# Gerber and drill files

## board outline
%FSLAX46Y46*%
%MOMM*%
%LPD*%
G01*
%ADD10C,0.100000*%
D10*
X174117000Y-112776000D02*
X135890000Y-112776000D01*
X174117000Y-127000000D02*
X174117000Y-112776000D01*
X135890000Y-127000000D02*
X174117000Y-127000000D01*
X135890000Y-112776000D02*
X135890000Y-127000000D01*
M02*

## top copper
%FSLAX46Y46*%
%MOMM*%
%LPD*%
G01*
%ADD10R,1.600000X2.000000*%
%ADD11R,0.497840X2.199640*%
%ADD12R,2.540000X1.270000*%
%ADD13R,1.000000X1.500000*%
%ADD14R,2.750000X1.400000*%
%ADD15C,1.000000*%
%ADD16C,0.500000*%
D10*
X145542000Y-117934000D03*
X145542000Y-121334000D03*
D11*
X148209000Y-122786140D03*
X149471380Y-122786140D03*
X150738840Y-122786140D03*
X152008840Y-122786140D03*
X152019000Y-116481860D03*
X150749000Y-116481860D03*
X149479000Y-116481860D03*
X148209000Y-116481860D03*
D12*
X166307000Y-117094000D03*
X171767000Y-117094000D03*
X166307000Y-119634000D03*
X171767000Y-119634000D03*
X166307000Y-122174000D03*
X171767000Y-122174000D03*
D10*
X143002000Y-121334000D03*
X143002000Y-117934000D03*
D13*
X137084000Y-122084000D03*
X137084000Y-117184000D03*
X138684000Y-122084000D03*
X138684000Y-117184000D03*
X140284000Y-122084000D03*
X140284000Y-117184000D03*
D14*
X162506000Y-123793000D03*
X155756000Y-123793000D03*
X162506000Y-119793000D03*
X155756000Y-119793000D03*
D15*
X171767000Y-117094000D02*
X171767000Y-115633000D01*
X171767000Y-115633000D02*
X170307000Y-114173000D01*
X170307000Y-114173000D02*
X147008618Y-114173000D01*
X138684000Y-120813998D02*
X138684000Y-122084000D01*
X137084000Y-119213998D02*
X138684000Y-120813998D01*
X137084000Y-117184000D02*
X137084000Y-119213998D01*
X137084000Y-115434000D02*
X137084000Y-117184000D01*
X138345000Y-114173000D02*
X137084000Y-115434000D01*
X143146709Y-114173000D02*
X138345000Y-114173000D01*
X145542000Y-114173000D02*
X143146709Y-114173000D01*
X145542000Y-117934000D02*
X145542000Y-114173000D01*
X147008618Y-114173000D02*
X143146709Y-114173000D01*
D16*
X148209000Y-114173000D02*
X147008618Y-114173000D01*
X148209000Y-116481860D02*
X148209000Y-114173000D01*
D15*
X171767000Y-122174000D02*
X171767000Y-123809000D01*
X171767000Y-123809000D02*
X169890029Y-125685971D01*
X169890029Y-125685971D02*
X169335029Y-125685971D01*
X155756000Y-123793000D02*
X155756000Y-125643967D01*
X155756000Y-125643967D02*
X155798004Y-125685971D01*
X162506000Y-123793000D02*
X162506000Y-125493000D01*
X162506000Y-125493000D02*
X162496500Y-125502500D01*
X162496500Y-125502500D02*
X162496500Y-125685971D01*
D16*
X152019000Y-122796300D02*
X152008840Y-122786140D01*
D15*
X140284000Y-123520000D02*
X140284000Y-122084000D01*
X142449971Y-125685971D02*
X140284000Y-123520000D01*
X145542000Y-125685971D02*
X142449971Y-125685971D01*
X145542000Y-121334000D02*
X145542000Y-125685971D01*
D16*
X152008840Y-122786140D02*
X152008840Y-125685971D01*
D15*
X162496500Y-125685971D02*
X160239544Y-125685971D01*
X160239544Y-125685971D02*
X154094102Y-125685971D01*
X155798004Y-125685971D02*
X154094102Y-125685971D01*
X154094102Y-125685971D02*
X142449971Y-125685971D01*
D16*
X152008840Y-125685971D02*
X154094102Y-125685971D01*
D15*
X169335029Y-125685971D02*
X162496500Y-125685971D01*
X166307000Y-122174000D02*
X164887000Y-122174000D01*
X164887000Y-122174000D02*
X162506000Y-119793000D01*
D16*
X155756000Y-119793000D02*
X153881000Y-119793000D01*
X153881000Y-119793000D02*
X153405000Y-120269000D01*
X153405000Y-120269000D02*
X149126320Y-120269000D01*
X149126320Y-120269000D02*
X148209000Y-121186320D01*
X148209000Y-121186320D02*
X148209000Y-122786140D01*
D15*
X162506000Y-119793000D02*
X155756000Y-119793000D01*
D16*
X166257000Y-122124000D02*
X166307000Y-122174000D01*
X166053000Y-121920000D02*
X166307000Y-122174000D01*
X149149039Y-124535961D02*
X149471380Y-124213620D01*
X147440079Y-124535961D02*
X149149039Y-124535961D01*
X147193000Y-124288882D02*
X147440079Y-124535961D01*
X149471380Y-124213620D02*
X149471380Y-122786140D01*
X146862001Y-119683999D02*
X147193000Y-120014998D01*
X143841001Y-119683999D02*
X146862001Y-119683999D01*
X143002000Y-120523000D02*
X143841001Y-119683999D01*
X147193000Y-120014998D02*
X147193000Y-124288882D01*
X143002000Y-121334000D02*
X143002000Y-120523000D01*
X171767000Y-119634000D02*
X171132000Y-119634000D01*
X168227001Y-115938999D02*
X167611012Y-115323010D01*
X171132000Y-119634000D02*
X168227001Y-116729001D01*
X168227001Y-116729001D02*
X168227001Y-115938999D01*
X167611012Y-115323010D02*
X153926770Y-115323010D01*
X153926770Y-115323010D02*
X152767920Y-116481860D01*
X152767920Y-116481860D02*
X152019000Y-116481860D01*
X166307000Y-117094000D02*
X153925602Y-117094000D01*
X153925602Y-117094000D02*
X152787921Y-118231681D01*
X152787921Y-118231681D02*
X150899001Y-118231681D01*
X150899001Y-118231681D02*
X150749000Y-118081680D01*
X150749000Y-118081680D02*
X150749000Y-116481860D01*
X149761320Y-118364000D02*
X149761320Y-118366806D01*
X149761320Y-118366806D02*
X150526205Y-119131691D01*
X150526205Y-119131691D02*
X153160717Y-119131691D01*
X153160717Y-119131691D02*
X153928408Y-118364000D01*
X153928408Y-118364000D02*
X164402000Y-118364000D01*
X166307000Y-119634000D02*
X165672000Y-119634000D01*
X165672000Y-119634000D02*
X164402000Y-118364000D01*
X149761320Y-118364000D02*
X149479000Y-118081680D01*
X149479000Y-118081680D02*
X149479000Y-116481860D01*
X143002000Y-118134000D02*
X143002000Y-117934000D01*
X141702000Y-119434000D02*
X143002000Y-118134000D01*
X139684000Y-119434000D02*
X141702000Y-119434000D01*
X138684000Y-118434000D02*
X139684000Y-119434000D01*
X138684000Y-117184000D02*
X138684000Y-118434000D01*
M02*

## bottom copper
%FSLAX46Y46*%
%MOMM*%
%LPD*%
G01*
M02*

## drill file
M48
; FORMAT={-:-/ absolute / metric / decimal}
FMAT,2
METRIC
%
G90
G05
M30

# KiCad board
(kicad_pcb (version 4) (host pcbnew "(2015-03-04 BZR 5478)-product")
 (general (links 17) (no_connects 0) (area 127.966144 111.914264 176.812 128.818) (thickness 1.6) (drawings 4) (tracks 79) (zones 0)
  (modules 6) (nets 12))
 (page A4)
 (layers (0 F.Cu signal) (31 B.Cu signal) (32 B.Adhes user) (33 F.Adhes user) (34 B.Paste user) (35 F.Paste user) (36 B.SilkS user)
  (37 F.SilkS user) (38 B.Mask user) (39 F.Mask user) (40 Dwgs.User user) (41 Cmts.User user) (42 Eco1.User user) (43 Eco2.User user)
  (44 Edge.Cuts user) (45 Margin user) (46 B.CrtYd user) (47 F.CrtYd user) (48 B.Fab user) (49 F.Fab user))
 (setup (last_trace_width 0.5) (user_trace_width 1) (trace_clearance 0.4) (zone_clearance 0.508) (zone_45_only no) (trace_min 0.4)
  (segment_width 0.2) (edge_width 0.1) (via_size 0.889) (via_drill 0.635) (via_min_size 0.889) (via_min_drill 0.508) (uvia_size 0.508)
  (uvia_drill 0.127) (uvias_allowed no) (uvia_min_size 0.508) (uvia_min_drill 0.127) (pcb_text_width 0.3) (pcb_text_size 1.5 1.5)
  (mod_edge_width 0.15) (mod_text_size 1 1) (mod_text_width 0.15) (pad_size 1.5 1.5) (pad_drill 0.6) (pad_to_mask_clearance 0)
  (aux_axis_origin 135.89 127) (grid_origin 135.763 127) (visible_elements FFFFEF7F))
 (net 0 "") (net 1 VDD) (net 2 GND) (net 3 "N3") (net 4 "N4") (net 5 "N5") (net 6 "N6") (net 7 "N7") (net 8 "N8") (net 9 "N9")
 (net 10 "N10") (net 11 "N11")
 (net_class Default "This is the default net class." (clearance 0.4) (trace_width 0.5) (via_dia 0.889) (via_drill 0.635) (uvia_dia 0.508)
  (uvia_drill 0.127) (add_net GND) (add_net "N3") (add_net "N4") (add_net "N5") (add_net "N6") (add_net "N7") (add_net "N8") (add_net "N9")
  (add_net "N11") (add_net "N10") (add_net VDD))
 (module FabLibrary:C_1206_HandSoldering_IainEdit (layer F.Cu) (at 145.542 119.634 270)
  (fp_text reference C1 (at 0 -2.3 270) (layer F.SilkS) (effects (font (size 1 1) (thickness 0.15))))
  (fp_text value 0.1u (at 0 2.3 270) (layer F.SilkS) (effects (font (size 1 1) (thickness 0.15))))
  (pad 1 smd rect (at -1.7 0 270) (size 2 1.6) (layers F.Cu F.Paste F.Mask) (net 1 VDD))
  (pad 2 smd rect (at 1.7 0 270) (size 2 1.6) (layers F.Cu F.Paste F.Mask) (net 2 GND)))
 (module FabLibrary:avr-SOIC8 (layer F.Cu) (at 150.114 119.634)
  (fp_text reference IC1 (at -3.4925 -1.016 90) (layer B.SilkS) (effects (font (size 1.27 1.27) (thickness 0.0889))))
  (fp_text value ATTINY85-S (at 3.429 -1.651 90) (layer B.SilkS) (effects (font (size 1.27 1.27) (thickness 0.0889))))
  (pad 1 smd rect (at -1.905 3.15214) (size 0.49784 2.19964) (layers F.Cu F.Paste F.Mask) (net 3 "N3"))
  (pad 2 smd rect (at -0.64262 3.15214) (size 0.49784 2.19964) (layers F.Cu F.Paste F.Mask) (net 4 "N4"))
  (pad 3 smd rect (at 0.62484 3.15214) (size 0.49784 2.19964) (layers F.Cu F.Paste F.Mask) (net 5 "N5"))
  (pad 4 smd rect (at 1.89484 3.15214) (size 0.49784 2.19964) (layers F.Cu F.Paste F.Mask) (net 2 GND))
  (pad 5 smd rect (at 1.905 -3.15214) (size 0.49784 2.19964) (layers F.Cu F.Paste F.Mask) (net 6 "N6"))
  (pad 6 smd rect (at 0.635 -3.15214) (size 0.49784 2.19964) (layers F.Cu F.Paste F.Mask) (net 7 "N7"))
  (pad 7 smd rect (at -0.635 -3.15214) (size 0.49784 2.19964) (layers F.Cu F.Paste F.Mask) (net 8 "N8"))
  (pad 8 smd rect (at -1.905 -3.15214) (size 0.49784 2.19964) (layers F.Cu F.Paste F.Mask) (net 1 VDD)))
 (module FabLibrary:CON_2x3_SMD (layer F.Cu) (at 169.037 119.634)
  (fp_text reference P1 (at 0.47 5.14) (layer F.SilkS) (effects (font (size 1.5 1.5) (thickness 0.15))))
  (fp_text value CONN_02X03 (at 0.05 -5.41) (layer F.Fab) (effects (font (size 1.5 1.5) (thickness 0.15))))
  (pad 1 smd rect (at -2.73 -2.54) (size 2.54 1.27) (layers F.Cu F.Paste F.Mask) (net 7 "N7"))
  (pad 2 smd rect (at 2.73 -2.54) (size 2.54 1.27) (layers F.Cu F.Paste F.Mask) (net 1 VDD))
  (pad 3 smd rect (at -2.73 0) (size 2.54 1.27) (layers F.Cu F.Paste F.Mask) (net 8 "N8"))
  (pad 4 smd rect (at 2.73 0) (size 2.54 1.27) (layers F.Cu F.Paste F.Mask) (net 6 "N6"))
  (pad 5 smd rect (at -2.73 2.54) (size 2.54 1.27) (layers F.Cu F.Paste F.Mask) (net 3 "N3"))
  (pad 6 smd rect (at 2.73 2.54) (size 2.54 1.27) (layers F.Cu F.Paste F.Mask) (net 2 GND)))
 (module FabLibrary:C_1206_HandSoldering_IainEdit (layer F.Cu) (at 143.002 119.634 90)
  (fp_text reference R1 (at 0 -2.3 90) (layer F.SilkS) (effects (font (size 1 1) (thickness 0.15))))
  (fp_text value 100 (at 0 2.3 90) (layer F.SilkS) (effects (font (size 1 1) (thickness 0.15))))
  (pad 1 smd rect (at -1.7 0 90) (size 2 1.6) (layers F.Cu F.Paste F.Mask) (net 4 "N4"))
  (pad 2 smd rect (at 1.7 0 90) (size 2 1.6) (layers F.Cu F.Paste F.Mask) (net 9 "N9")))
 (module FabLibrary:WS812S (layer F.Cu) (at 138.684 119.634 90)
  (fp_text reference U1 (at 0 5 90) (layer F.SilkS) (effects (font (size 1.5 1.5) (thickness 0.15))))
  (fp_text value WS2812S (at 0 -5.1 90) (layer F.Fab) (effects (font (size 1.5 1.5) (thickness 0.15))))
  (pad 4 smd rect (at -2.45 -1.6 90) (size 1.5 1) (layers F.Cu F.Paste F.Mask) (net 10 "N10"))
  (pad 3 smd rect (at 2.45 -1.6 90) (size 1.5 1) (layers F.Cu F.Paste F.Mask) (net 1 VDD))
  (pad 5 smd rect (at -2.45 0 90) (size 1.5 1) (layers F.Cu F.Paste F.Mask) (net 1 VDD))
  (pad 2 smd rect (at 2.45 0 90) (size 1.5 1) (layers F.Cu F.Paste F.Mask) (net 9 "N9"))
  (pad 6 smd rect (at -2.45 1.6 90) (size 1.5 1) (layers F.Cu F.Paste F.Mask) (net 2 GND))
  (pad 1 smd rect (at 2.45 1.6 90) (size 1.5 1) (layers F.Cu F.Paste F.Mask) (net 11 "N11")))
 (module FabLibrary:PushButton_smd (layer F.Cu) (at 159.131 121.793 180)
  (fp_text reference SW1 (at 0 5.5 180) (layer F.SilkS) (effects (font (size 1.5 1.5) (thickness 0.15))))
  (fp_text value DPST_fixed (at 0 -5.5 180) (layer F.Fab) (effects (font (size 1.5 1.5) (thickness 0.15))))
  (pad 4 smd rect (at -3.375 -2 180) (size 2.75 1.4) (layers F.Cu F.Paste F.Mask) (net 2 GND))
  (pad 3 smd rect (at 3.375 -2 180) (size 2.75 1.4) (layers F.Cu F.Paste F.Mask) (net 2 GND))
  (pad 2 smd rect (at -3.375 2 180) (size 2.75 1.4) (layers F.Cu F.Paste F.Mask) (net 3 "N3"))
  (pad 1 smd rect (at 3.375 2 180) (size 2.75 1.4) (layers F.Cu F.Paste F.Mask) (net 3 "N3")))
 (gr_line (start 174.117 112.776) (end 135.89 112.776) (layer Edge.Cuts) (width 0.1))
 (gr_line (start 174.117 127) (end 174.117 112.776) (layer Edge.Cuts) (width 0.1))
 (gr_line (start 135.89 127) (end 174.117 127) (layer Edge.Cuts) (width 0.1))
 (gr_line (start 135.89 112.776) (end 135.89 127) (angle 90) (layer Edge.Cuts) (width 0.1))
 (segment (start 171.767 117.094) (end 171.767 115.633) (width 1) (layer F.Cu) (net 1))
 (segment (start 171.767 115.633) (end 170.307 114.173) (width 1) (layer F.Cu) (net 1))
 (segment (start 170.307 114.173) (end 147.008618 114.173) (width 1) (layer F.Cu) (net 1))
 (segment (start 138.684 120.813998) (end 138.684 122.084) (width 1) (layer F.Cu) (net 1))
 (segment (start 137.084 119.213998) (end 138.684 120.813998) (width 1) (layer F.Cu) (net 1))
 (segment (start 137.084 117.184) (end 137.084 119.213998) (width 1) (layer F.Cu) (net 1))
 (segment (start 137.084 115.434) (end 137.084 117.184) (width 1) (layer F.Cu) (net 1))
 (segment (start 138.345 114.173) (end 137.084 115.434) (width 1) (layer F.Cu) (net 1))
 (segment (start 143.146709 114.173) (end 138.345 114.173) (width 1) (layer F.Cu) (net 1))
 (segment (start 145.542 114.173) (end 143.146709 114.173) (width 1) (layer F.Cu) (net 1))
 (segment (start 145.542 117.934) (end 145.542 114.173) (width 1) (layer F.Cu) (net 1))
 (segment (start 147.008618 114.173) (end 143.146709 114.173) (width 1) (layer F.Cu) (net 1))
 (segment (start 148.209 114.173) (end 147.008618 114.173) (width 0.5) (layer F.Cu) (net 1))
 (segment (start 148.209 116.48186) (end 148.209 114.173) (width 0.5) (layer F.Cu) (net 1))
 (segment (start 171.767 122.174) (end 171.767 123.809) (width 1) (layer F.Cu) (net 2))
 (segment (start 171.767 123.809) (end 169.890029 125.685971) (width 1) (layer F.Cu) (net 2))
 (segment (start 169.890029 125.685971) (end 169.335029 125.685971) (width 1) (layer F.Cu) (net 2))
 (segment (start 155.756 123.793) (end 155.756 125.643967) (width 1) (layer F.Cu) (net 2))
 (segment (start 155.756 125.643967) (end 155.798004 125.685971) (width 1) (layer F.Cu) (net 2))
 (segment (start 162.506 123.793) (end 162.506 125.493) (width 1) (layer F.Cu) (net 2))
 (segment (start 162.506 125.493) (end 162.4965 125.5025) (width 1) (layer F.Cu) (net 2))
 (segment (start 162.4965 125.5025) (end 162.4965 125.685971) (width 1) (layer F.Cu) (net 2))
 (segment (start 152.019 122.7963) (end 152.00884 122.78614) (width 0.5) (layer F.Cu) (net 2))
 (segment (start 140.284 123.52) (end 140.284 122.084) (width 1) (layer F.Cu) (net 2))
 (segment (start 142.449971 125.685971) (end 140.284 123.52) (width 1) (layer F.Cu) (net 2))
 (segment (start 145.542 125.685971) (end 142.449971 125.685971) (width 1) (layer F.Cu) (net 2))
 (segment (start 145.542 121.334) (end 145.542 125.685971) (width 1) (layer F.Cu) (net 2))
 (segment (start 152.00884 122.78614) (end 152.00884 125.685971) (width 0.5) (layer F.Cu) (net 2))
 (segment (start 162.4965 125.685971) (end 160.239544 125.685971) (width 1) (layer F.Cu) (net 2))
 (segment (start 160.239544 125.685971) (end 154.094102 125.685971) (width 1) (layer F.Cu) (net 2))
 (segment (start 155.798004 125.685971) (end 154.094102 125.685971) (width 1) (layer F.Cu) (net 2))
 (segment (start 154.094102 125.685971) (end 142.449971 125.685971) (width 1) (layer F.Cu) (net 2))
 (segment (start 152.00884 125.685971) (end 154.094102 125.685971) (width 0.5) (layer F.Cu) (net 2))
 (segment (start 169.335029 125.685971) (end 162.4965 125.685971) (width 1) (layer F.Cu) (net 2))
 (segment (start 166.307 122.174) (end 164.887 122.174) (width 1) (layer F.Cu) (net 3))
 (segment (start 164.887 122.174) (end 162.506 119.793) (width 1) (layer F.Cu) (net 3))
 (segment (start 155.756 119.793) (end 153.881 119.793) (width 0.5) (layer F.Cu) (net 3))
 (segment (start 153.881 119.793) (end 153.405 120.269) (width 0.5) (layer F.Cu) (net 3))
 (segment (start 153.405 120.269) (end 149.12632 120.269) (width 0.5) (layer F.Cu) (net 3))
 (segment (start 149.12632 120.269) (end 148.209 121.18632) (width 0.5) (layer F.Cu) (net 3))
 (segment (start 148.209 121.18632) (end 148.209 122.78614) (width 0.5) (layer F.Cu) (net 3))
 (segment (start 162.506 119.793) (end 155.756 119.793) (width 1) (layer F.Cu) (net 3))
 (segment (start 166.257 122.124) (end 166.307 122.174) (width 0.5) (layer F.Cu) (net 3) (status 30))
 (segment (start 166.053 121.92) (end 166.307 122.174) (width 0.5) (layer F.Cu) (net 3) (status 30))
 (segment (start 149.149039 124.535961) (end 149.47138 124.21362) (width 0.5) (layer F.Cu) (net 4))
 (segment (start 147.440079 124.535961) (end 149.149039 124.535961) (width 0.5) (layer F.Cu) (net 4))
 (segment (start 147.193 124.288882) (end 147.440079 124.535961) (width 0.5) (layer F.Cu) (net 4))
 (segment (start 149.47138 124.21362) (end 149.47138 122.78614) (width 0.5) (layer F.Cu) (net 4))
 (segment (start 146.862001 119.683999) (end 147.193 120.014998) (width 0.5) (layer F.Cu) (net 4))
 (segment (start 143.841001 119.683999) (end 146.862001 119.683999) (width 0.5) (layer F.Cu) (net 4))
 (segment (start 143.002 120.523) (end 143.841001 119.683999) (width 0.5) (layer F.Cu) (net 4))
 (segment (start 147.193 120.014998) (end 147.193 124.288882) (width 0.5) (layer F.Cu) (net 4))
 (segment (start 143.002 121.334) (end 143.002 120.523) (width 0.5) (layer F.Cu) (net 4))
 (segment (start 171.767 119.634) (end 171.132 119.634) (width 0.5) (layer F.Cu) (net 6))
 (segment (start 168.227001 115.938999) (end 167.611012 115.32301) (width 0.5) (layer F.Cu) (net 6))
 (segment (start 171.132 119.634) (end 168.227001 116.729001) (width 0.5) (layer F.Cu) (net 6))
 (segment (start 168.227001 116.729001) (end 168.227001 115.938999) (width 0.5) (layer F.Cu) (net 6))
 (segment (start 167.611012 115.32301) (end 153.92677 115.32301) (width 0.5) (layer F.Cu) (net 6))
 (segment (start 153.92677 115.32301) (end 152.76792 116.48186) (width 0.5) (layer F.Cu) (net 6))
 (segment (start 152.76792 116.48186) (end 152.019 116.48186) (width 0.5) (layer F.Cu) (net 6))
 (segment (start 166.307 117.094) (end 153.925602 117.094) (width 0.5) (layer F.Cu) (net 7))
 (segment (start 153.925602 117.094) (end 152.787921 118.231681) (width 0.5) (layer F.Cu) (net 7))
 (segment (start 152.787921 118.231681) (end 150.899001 118.231681) (width 0.5) (layer F.Cu) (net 7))
 (segment (start 150.899001 118.231681) (end 150.749 118.08168) (width 0.5) (layer F.Cu) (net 7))
 (segment (start 150.749 118.08168) (end 150.749 116.48186) (width 0.5) (layer F.Cu) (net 7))
 (segment (start 149.76132 118.364) (end 149.76132 118.366806) (width 0.5) (layer F.Cu) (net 8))
 (segment (start 149.76132 118.366806) (end 150.526205 119.131691) (width 0.5) (layer F.Cu) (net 8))
 (segment (start 150.526205 119.131691) (end 153.160717 119.131691) (width 0.5) (layer F.Cu) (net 8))
 (segment (start 153.160717 119.131691) (end 153.928408 118.364) (width 0.5) (layer F.Cu) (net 8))
 (segment (start 153.928408 118.364) (end 164.402 118.364) (width 0.5) (layer F.Cu) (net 8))
 (segment (start 166.307 119.634) (end 165.672 119.634) (width 0.5) (layer F.Cu) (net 8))
 (segment (start 165.672 119.634) (end 164.402 118.364) (width 0.5) (layer F.Cu) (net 8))
 (segment (start 149.76132 118.364) (end 149.479 118.08168) (width 0.5) (layer F.Cu) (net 8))
 (segment (start 149.479 118.08168) (end 149.479 116.48186) (width 0.5) (layer F.Cu) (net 8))
 (segment (start 143.002 118.134) (end 143.002 117.934) (width 0.5) (layer F.Cu) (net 9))
 (segment (start 141.702 119.434) (end 143.002 118.134) (width 0.5) (layer F.Cu) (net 9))
 (segment (start 139.684 119.434) (end 141.702 119.434) (width 0.5) (layer F.Cu) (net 9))
 (segment (start 138.684 118.434) (end 139.684 119.434) (width 0.5) (layer F.Cu) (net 9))
 (segment (start 138.684 117.184) (end 138.684 118.434) (width 0.5) (layer F.Cu) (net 9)))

